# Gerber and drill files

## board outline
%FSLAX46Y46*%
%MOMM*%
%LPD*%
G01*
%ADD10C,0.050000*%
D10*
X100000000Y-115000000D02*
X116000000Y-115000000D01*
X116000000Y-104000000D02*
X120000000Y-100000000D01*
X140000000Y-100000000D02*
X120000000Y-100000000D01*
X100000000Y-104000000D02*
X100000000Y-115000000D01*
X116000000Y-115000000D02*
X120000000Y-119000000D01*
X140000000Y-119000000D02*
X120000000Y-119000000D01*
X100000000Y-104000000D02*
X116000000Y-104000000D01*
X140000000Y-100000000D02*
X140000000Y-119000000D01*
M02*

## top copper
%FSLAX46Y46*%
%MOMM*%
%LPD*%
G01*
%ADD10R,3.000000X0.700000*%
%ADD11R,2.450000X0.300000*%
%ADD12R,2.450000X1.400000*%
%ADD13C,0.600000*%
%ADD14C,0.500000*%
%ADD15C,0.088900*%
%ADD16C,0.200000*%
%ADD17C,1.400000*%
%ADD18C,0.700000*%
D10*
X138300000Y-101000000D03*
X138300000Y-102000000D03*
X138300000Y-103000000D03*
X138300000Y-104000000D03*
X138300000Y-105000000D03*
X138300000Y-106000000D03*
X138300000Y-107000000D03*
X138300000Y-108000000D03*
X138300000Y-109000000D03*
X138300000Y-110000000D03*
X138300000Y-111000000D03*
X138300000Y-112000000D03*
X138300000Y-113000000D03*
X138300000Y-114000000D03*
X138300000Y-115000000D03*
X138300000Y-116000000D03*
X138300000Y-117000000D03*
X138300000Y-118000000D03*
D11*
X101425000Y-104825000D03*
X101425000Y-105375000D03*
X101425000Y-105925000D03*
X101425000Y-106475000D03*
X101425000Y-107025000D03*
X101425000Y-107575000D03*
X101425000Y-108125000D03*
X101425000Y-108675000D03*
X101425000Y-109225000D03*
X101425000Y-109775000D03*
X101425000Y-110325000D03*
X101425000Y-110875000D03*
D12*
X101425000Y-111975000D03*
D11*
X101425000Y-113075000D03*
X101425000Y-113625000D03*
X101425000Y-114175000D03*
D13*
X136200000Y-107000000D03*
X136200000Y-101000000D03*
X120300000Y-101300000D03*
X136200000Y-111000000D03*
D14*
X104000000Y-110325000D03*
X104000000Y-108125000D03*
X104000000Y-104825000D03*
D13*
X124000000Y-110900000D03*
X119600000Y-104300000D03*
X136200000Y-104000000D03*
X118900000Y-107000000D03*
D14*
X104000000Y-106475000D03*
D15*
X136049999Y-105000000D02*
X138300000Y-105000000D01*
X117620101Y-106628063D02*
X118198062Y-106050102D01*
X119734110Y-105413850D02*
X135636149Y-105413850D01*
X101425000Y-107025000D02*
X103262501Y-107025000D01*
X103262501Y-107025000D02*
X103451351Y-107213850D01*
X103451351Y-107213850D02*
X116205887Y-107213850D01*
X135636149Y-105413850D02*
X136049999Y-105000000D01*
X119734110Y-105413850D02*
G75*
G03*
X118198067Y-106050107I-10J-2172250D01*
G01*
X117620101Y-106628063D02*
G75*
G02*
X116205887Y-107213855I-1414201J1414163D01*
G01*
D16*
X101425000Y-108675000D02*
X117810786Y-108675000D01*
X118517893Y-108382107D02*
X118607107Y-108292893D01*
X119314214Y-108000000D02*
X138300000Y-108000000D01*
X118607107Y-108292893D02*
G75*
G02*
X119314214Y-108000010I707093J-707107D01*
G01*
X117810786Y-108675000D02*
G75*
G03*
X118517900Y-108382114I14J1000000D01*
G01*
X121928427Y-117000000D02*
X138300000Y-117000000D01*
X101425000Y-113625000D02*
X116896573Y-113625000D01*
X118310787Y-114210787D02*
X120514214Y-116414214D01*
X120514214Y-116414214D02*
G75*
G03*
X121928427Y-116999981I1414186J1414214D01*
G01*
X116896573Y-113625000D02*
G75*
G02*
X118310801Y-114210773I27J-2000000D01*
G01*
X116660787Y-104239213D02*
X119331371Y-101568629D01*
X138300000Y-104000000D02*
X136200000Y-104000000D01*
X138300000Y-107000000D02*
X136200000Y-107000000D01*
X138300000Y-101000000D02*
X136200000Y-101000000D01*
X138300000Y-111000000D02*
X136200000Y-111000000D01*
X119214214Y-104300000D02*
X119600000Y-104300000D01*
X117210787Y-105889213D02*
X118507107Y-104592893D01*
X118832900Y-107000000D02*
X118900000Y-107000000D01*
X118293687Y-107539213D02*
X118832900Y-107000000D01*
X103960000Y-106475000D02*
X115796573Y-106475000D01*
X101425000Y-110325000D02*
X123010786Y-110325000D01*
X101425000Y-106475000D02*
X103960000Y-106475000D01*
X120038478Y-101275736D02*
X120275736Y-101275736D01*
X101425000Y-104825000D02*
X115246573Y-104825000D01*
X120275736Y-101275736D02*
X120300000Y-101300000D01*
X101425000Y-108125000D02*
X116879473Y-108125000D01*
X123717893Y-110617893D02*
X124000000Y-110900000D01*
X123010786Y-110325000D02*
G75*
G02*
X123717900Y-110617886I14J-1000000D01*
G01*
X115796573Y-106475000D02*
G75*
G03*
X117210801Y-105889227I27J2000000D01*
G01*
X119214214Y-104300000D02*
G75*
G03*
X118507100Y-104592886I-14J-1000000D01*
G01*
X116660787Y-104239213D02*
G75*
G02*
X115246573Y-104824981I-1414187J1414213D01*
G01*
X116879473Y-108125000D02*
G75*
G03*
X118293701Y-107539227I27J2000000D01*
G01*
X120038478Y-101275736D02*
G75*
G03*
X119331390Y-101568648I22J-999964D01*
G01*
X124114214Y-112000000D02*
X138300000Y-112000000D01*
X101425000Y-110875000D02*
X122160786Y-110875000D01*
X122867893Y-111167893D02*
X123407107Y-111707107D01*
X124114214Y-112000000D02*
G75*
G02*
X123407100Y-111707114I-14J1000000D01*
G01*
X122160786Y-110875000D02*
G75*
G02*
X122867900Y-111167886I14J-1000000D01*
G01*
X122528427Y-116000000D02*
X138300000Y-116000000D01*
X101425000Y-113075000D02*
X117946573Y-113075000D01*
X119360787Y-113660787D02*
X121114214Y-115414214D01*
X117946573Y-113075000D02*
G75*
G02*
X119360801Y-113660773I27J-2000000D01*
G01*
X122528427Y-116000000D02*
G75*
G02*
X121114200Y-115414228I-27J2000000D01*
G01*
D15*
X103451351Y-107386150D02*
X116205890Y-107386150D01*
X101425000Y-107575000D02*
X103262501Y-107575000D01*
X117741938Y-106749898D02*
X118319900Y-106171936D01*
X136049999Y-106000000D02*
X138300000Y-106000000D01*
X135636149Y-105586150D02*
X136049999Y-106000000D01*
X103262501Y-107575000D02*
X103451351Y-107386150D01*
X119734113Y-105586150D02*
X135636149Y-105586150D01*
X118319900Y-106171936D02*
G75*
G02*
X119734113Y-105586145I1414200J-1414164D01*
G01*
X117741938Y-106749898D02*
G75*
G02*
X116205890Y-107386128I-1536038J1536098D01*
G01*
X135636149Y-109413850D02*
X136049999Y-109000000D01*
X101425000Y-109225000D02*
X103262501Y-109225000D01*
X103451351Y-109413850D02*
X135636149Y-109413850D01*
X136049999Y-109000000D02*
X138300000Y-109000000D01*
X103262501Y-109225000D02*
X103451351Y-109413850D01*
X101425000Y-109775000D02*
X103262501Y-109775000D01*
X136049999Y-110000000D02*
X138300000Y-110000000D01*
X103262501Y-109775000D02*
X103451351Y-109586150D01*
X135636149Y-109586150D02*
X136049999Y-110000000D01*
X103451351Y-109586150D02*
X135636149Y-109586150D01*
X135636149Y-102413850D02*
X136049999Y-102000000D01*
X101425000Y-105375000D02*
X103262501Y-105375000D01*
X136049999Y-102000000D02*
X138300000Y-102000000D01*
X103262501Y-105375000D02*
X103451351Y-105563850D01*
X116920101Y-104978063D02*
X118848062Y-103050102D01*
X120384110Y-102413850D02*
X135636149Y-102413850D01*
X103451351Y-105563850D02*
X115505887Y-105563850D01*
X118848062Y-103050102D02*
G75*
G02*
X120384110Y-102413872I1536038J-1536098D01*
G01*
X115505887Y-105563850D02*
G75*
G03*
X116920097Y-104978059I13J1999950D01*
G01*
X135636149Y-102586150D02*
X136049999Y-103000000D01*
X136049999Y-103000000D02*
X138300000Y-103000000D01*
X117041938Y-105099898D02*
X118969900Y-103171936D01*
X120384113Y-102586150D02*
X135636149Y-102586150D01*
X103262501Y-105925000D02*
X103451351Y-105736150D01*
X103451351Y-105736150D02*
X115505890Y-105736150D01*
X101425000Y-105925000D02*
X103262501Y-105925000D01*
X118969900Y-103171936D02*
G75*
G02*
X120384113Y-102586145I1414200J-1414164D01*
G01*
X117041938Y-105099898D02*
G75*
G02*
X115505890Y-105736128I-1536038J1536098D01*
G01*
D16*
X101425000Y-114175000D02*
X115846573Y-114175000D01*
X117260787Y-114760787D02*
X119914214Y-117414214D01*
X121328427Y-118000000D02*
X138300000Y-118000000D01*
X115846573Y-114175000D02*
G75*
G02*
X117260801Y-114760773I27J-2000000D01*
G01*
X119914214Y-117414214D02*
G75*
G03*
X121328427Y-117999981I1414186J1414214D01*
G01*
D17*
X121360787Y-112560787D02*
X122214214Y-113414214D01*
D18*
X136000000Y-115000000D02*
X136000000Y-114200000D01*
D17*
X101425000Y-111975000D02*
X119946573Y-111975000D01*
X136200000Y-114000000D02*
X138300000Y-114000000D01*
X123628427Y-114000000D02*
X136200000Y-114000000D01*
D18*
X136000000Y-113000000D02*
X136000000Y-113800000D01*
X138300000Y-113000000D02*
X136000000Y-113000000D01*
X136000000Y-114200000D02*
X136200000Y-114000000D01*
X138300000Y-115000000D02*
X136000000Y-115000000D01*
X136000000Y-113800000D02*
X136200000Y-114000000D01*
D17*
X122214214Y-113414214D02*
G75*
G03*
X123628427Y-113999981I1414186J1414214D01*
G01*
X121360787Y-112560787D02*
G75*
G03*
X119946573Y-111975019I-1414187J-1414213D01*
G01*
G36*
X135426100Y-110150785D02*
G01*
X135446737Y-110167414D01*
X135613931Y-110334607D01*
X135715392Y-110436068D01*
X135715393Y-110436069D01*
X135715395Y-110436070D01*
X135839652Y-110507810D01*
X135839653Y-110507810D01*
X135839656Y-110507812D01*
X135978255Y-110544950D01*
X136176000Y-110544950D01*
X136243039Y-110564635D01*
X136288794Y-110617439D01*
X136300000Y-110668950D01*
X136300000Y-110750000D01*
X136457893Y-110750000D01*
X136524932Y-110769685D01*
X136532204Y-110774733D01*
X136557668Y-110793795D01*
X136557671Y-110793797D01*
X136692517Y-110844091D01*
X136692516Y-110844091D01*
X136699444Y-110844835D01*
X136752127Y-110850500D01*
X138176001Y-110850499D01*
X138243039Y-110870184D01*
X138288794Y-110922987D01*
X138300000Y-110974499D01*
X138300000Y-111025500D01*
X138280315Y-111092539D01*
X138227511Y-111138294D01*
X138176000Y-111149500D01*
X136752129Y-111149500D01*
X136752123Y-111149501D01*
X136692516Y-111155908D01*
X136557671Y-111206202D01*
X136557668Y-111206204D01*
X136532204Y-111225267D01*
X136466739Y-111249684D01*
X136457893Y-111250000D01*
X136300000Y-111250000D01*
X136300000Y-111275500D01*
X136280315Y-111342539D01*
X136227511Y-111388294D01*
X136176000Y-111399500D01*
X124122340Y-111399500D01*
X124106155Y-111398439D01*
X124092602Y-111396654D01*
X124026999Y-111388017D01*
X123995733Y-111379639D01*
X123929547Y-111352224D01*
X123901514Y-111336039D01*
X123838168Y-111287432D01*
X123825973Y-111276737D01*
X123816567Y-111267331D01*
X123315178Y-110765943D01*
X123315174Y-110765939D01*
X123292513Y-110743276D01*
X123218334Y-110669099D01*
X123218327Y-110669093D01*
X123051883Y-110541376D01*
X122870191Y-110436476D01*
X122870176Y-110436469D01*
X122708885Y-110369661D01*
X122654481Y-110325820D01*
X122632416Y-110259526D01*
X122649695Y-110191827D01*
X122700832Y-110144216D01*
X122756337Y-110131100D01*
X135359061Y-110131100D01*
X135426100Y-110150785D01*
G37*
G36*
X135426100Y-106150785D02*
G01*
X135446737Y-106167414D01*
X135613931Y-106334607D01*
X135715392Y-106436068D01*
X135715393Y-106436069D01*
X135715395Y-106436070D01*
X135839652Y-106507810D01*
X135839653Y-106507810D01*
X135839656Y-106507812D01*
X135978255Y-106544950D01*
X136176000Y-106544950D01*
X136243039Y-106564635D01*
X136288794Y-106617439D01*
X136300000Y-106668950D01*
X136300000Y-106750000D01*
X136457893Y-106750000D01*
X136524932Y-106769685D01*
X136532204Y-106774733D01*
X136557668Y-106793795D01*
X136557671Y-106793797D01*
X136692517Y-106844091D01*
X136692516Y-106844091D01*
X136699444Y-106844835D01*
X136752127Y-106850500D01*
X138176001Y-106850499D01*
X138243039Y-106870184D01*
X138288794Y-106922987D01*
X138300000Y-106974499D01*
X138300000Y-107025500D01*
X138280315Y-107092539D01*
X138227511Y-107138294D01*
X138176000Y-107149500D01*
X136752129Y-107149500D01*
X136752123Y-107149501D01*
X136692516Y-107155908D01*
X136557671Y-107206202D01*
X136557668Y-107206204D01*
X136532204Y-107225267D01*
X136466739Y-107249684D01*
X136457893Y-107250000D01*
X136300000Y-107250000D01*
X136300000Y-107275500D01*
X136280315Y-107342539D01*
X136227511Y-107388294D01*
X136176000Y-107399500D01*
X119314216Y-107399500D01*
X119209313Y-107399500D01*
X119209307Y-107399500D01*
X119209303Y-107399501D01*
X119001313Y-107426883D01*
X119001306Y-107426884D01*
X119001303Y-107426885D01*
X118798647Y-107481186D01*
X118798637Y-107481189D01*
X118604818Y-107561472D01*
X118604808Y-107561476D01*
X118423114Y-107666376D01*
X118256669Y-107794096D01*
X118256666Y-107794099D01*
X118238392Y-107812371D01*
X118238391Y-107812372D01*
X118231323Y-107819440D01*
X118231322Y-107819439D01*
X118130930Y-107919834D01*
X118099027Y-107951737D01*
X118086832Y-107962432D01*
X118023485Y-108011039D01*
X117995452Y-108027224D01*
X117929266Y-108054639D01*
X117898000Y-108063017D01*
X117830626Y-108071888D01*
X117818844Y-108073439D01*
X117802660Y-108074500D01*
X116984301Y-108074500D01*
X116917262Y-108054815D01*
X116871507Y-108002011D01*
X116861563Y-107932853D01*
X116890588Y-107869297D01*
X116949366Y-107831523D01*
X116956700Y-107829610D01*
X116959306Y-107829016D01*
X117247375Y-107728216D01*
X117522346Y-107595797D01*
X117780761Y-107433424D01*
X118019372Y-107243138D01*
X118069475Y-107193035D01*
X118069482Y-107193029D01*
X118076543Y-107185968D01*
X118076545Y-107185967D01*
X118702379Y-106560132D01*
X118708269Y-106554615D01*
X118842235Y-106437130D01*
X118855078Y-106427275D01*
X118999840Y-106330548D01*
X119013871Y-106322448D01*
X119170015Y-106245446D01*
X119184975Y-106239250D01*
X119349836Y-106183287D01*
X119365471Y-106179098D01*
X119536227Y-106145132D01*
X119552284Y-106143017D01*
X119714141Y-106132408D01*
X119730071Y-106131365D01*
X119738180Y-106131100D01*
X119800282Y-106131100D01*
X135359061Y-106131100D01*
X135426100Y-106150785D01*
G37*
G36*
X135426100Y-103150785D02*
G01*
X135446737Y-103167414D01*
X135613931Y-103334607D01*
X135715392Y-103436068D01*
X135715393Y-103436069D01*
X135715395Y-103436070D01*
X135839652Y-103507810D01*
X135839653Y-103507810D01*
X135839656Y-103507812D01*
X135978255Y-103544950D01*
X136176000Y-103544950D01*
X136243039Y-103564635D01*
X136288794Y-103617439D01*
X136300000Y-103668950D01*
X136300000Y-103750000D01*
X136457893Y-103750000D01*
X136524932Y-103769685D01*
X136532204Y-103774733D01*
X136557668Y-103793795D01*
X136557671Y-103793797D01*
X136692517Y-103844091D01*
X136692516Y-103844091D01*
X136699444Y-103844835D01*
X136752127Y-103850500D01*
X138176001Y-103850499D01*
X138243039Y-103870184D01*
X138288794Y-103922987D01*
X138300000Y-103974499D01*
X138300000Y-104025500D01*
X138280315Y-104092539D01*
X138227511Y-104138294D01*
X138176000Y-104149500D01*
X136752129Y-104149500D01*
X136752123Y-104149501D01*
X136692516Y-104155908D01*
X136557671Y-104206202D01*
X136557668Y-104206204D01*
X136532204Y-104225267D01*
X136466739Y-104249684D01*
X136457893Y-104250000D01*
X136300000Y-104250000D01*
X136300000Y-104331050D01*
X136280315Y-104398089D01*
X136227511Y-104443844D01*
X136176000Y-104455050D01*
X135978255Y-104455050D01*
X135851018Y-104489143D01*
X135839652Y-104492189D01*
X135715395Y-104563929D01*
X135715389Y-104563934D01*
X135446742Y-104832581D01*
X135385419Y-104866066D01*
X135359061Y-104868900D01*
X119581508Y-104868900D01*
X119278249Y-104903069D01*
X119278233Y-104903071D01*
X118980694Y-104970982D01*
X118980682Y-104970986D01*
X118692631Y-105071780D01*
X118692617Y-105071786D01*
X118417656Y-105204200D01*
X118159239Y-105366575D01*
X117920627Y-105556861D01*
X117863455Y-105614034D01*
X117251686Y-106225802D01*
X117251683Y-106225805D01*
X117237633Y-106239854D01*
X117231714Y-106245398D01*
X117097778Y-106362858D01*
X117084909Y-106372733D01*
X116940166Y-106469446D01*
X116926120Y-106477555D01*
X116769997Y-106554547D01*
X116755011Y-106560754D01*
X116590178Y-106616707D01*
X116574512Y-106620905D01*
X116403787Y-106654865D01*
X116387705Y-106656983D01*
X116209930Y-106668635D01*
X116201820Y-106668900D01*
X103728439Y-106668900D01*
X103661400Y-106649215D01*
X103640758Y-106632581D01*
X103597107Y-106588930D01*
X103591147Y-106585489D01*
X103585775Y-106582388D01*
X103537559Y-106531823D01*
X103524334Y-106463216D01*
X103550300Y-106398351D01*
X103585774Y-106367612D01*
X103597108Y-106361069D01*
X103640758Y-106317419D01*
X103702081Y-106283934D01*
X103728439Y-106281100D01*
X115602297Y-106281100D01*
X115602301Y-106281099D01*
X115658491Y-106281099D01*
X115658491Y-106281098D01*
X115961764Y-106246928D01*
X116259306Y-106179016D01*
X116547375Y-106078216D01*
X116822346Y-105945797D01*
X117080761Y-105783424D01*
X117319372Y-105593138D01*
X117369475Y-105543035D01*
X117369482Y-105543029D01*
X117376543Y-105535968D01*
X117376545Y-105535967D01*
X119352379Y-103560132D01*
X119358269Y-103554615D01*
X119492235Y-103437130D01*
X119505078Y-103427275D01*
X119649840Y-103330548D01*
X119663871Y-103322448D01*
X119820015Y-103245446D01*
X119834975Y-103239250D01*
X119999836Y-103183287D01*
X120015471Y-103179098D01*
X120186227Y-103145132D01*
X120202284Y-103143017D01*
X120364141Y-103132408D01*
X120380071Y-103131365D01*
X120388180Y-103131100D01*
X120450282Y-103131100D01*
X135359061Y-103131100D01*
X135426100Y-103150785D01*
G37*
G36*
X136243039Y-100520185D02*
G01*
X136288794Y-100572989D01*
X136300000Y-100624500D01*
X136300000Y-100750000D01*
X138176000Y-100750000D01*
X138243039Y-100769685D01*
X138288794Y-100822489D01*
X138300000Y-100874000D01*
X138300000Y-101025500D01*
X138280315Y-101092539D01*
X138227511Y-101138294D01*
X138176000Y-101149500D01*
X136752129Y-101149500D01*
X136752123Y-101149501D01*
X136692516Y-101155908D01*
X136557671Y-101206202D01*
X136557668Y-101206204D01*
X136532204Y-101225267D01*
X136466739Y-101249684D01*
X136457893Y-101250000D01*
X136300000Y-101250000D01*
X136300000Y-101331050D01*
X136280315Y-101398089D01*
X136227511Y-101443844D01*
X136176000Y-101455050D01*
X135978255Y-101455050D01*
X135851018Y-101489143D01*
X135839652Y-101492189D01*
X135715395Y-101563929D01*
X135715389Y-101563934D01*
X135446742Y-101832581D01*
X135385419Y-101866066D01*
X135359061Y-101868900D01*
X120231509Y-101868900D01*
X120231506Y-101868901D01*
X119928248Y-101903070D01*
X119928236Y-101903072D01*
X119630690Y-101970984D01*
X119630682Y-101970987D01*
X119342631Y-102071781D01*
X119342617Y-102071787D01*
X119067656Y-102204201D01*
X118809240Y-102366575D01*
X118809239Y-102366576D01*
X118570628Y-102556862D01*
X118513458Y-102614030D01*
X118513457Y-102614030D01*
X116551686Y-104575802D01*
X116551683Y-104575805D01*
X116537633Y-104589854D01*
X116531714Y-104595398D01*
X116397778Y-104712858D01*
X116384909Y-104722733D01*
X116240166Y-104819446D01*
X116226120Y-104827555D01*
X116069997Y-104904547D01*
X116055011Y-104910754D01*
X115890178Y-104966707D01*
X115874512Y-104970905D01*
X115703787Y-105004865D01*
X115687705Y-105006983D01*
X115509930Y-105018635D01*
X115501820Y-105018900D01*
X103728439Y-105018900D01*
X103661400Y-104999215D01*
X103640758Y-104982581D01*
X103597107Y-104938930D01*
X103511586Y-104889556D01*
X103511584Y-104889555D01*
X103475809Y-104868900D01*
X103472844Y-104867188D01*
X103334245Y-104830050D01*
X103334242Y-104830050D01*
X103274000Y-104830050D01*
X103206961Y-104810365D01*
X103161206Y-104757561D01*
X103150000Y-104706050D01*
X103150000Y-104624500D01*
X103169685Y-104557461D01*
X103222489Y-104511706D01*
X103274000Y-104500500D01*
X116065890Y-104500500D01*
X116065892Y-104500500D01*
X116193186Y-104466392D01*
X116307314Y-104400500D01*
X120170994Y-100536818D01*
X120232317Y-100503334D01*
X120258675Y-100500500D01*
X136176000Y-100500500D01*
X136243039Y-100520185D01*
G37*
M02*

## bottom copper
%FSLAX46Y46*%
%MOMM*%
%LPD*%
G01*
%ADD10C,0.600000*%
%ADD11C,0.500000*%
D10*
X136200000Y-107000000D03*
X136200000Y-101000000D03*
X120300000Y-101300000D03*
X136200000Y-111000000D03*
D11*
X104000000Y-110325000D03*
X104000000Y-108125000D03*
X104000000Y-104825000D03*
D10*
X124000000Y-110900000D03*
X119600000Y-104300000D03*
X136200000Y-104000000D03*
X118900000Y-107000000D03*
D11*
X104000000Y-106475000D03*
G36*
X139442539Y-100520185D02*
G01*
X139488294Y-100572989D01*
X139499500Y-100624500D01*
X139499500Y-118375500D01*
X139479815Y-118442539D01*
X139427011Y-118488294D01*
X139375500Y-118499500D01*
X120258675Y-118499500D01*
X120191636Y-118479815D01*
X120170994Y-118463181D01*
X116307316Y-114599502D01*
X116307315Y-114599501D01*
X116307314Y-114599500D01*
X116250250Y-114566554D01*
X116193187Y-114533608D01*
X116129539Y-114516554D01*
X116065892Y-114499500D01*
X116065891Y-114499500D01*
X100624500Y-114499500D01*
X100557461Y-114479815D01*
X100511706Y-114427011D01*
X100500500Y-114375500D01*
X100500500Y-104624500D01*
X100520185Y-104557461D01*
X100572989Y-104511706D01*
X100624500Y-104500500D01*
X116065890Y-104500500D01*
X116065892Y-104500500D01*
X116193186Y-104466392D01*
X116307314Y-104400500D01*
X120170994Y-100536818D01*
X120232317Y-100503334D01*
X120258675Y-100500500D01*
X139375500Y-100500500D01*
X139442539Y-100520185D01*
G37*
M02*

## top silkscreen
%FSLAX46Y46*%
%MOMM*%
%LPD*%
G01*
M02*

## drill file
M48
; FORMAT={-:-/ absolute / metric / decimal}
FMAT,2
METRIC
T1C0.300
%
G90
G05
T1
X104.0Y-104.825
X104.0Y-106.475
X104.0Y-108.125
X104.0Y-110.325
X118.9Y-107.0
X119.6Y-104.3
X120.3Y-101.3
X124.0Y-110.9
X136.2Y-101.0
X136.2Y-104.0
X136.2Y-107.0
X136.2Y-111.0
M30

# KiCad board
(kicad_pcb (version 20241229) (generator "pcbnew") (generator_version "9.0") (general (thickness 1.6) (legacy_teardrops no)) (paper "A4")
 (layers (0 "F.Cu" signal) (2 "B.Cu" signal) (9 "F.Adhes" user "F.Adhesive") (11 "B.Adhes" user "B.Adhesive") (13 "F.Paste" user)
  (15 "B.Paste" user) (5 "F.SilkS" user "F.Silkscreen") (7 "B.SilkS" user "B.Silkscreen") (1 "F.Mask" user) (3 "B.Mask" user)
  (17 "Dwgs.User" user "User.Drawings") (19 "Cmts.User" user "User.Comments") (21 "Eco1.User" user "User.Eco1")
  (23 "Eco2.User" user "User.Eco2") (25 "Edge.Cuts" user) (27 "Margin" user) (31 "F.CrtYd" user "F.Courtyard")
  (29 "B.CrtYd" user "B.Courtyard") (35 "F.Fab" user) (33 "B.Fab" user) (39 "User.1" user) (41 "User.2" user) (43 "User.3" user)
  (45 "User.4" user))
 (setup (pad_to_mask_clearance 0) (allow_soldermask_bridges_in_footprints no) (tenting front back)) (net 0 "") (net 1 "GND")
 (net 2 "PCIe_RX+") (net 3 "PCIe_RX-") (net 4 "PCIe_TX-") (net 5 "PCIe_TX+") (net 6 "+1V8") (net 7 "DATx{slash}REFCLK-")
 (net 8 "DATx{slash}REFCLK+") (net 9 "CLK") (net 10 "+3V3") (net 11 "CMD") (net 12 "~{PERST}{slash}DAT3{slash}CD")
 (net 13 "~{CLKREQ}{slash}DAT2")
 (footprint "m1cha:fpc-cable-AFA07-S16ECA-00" (layer "F.Cu") (at 138.3 109.5 -90)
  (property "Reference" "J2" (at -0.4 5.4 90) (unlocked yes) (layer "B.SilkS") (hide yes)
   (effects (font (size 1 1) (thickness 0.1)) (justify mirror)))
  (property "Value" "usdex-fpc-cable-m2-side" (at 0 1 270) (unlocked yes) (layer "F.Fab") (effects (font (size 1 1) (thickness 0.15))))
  (pad "1" smd rect (at -8.5 0 270) (size 0.7 3) (layers "F.Cu" "F.Mask" "F.Paste") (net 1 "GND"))
  (pad "2" smd rect (at -7.5 0 270) (size 0.7 3) (layers "F.Cu" "F.Mask" "F.Paste") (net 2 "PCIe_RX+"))
  (pad "3" smd rect (at -6.5 0 270) (size 0.7 3) (layers "F.Cu" "F.Mask" "F.Paste") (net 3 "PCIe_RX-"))
  (pad "4" smd rect (at -5.5 0 270) (size 0.7 3) (layers "F.Cu" "F.Mask" "F.Paste") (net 1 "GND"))
  (pad "5" smd rect (at -4.5 0 270) (size 0.7 3) (layers "F.Cu" "F.Mask" "F.Paste") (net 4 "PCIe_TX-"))
  (pad "6" smd rect (at -3.5 0 270) (size 0.7 3) (layers "F.Cu" "F.Mask" "F.Paste") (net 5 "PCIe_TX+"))
  (pad "7" smd rect (at -2.5 0 270) (size 0.7 3) (layers "F.Cu" "F.Mask" "F.Paste") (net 1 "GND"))
  (pad "8" smd rect (at -1.5 0 270) (size 0.7 3) (layers "F.Cu" "F.Mask" "F.Paste") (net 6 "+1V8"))
  (pad "9" smd rect (at -0.5 0 270) (size 0.7 3) (layers "F.Cu" "F.Mask" "F.Paste") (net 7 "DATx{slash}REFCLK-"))
  (pad "10" smd rect (at 0.5 0 270) (size 0.7 3) (layers "F.Cu" "F.Mask" "F.Paste") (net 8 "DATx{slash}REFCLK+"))
  (pad "11" smd rect (at 1.5 0 270) (size 0.7 3) (layers "F.Cu" "F.Mask" "F.Paste") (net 1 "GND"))
  (pad "12" smd rect (at 2.5 0 270) (size 0.7 3) (layers "F.Cu" "F.Mask" "F.Paste") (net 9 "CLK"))
  (pad "13" smd rect (at 3.5 0 270) (size 0.7 3) (layers "F.Cu" "F.Mask" "F.Paste") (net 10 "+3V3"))
  (pad "14" smd rect (at 4.5 0 270) (size 0.7 3) (layers "F.Cu" "F.Mask" "F.Paste") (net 10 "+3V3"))
  (pad "15" smd rect (at 5.5 0 270) (size 0.7 3) (layers "F.Cu" "F.Mask" "F.Paste") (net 10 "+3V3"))
  (pad "16" smd rect (at 6.5 0 270) (size 0.7 3) (layers "F.Cu" "F.Mask" "F.Paste") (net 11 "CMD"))
  (pad "17" smd rect (at 7.5 0 270) (size 0.7 3) (layers "F.Cu" "F.Mask" "F.Paste") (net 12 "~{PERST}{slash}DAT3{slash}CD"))
  (pad "18" smd rect (at 8.5 0 270) (size 0.7 3) (layers "F.Cu" "F.Mask" "F.Paste") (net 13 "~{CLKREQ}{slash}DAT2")))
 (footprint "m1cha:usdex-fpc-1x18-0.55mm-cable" (layer "F.Cu") (at 101.425 109.5 -90)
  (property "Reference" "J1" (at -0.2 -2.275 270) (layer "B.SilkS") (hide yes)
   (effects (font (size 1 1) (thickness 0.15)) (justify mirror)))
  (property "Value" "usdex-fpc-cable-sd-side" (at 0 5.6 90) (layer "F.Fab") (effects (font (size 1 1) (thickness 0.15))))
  (pad "1" smd rect (at -4.675 0 270) (size 0.3 2.45) (layers "F.Cu" "F.Mask" "F.Paste") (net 1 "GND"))
  (pad "2" smd rect (at -4.125 0 270) (size 0.3 2.45) (layers "F.Cu" "F.Mask" "F.Paste") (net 2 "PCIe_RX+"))
  (pad "3" smd rect (at -3.575 0 270) (size 0.3 2.45) (layers "F.Cu" "F.Mask" "F.Paste") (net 3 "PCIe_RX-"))
  (pad "4" smd rect (at -3.025 0 270) (size 0.3 2.45) (layers "F.Cu" "F.Mask" "F.Paste") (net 1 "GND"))
  (pad "5" smd rect (at -2.475 0 270) (size 0.3 2.45) (layers "F.Cu" "F.Mask" "F.Paste") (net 4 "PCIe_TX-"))
  (pad "6" smd rect (at -1.925 0 270) (size 0.3 2.45) (layers "F.Cu" "F.Mask" "F.Paste") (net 5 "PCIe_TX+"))
  (pad "7" smd rect (at -1.375 0 270) (size 0.3 2.45) (layers "F.Cu" "F.Mask" "F.Paste") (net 1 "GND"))
  (pad "8" smd rect (at -0.825 0 270) (size 0.3 2.45) (layers "F.Cu" "F.Mask" "F.Paste") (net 6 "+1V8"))
  (pad "9" smd rect (at -0.275 0 270) (size 0.3 2.45) (layers "F.Cu" "F.Mask" "F.Paste") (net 7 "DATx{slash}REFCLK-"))
  (pad "10" smd rect (at 0.275 0 270) (size 0.3 2.45) (layers "F.Cu" "F.Mask" "F.Paste") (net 8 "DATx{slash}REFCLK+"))
  (pad "11" smd rect (at 0.825 0 270) (size 0.3 2.45) (layers "F.Cu" "F.Mask" "F.Paste") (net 1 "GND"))
  (pad "12" smd rect (at 1.375 0 270) (size 0.3 2.45) (layers "F.Cu" "F.Mask" "F.Paste") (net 9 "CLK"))
  (pad "13" smd rect (at 2.475 0 270) (size 1.4 2.45) (layers "F.Cu" "F.Mask" "F.Paste") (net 10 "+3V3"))
  (pad "14" smd rect (at 3.575 0 270) (size 0.3 2.45) (layers "F.Cu" "F.Mask" "F.Paste") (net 11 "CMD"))
  (pad "15" smd rect (at 4.125 0 270) (size 0.3 2.45) (layers "F.Cu" "F.Mask" "F.Paste") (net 12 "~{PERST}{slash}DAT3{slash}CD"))
  (pad "16" smd rect (at 4.675 0 270) (size 0.3 2.45) (layers "F.Cu" "F.Mask" "F.Paste") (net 13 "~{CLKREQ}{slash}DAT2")))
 (gr_line (start 100 115) (end 116 115) (stroke (width 0.05) (type solid)) (layer "Edge.Cuts"))
 (gr_line (start 116 104) (end 120 100) (stroke (width 0.05) (type default)) (layer "Edge.Cuts"))
 (gr_line (start 140 100) (end 120 100) (stroke (width 0.05) (type solid)) (layer "Edge.Cuts"))
 (gr_line (start 100 104) (end 100 115) (stroke (width 0.05) (type solid)) (layer "Edge.Cuts"))
 (gr_line (start 116 115) (end 120 119) (stroke (width 0.05) (type default)) (layer "Edge.Cuts"))
 (gr_line (start 140 119) (end 120 119) (stroke (width 0.05) (type solid)) (layer "Edge.Cuts"))
 (gr_line (start 100 104) (end 116 104) (stroke (width 0.05) (type solid)) (layer "Edge.Cuts"))
 (gr_line (start 140 100) (end 140 119) (stroke (width 0.05) (type default)) (layer "Edge.Cuts"))
 (segment (start 136.049999 105) (end 138.3 105) (width 0.0889) (layer "F.Cu") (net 4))
 (segment (start 117.620101 106.628063) (end 118.198062 106.050102) (width 0.0889) (layer "F.Cu") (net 4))
 (segment (start 119.73411 105.41385) (end 135.636149 105.41385) (width 0.0889) (layer "F.Cu") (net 4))
 (segment (start 101.425 107.025) (end 103.262501 107.025) (width 0.0889) (layer "F.Cu") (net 4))
 (segment (start 103.262501 107.025) (end 103.451351 107.21385) (width 0.0889) (layer "F.Cu") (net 4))
 (segment (start 103.451351 107.21385) (end 116.205887 107.21385) (width 0.0889) (layer "F.Cu") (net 4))
 (segment (start 135.636149 105.41385) (end 136.049999 105) (width 0.0889) (layer "F.Cu") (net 4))
 (arc (start 119.73411 105.41385) (mid 118.902807 105.579206) (end 118.198062 106.050102) (width 0.0889) (layer "F.Cu") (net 4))
 (arc (start 117.620101 106.628063) (mid 116.971254 107.061609) (end 116.205887 107.21385) (width 0.0889) (layer "F.Cu") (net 4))
 (segment (start 101.425 108.675) (end 117.810786 108.675) (width 0.2) (layer "F.Cu") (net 6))
 (segment (start 118.517893 108.382107) (end 118.607107 108.292893) (width 0.2) (layer "F.Cu") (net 6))
 (segment (start 119.314214 108) (end 138.3 108) (width 0.2) (layer "F.Cu") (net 6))
 (arc (start 118.607107 108.292893) (mid 118.93153 108.07612) (end 119.314214 108) (width 0.2) (layer "F.Cu") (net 6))
 (arc (start 117.810786 108.675) (mid 118.193469 108.59888) (end 118.517893 108.382107) (width 0.2) (layer "F.Cu") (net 6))
 (segment (start 121.928427 117) (end 138.3 117) (width 0.2) (layer "F.Cu") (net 12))
 (segment (start 101.425 113.625) (end 116.896573 113.625) (width 0.2) (layer "F.Cu") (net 12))
 (segment (start 118.310787 114.210787) (end 120.514214 116.414214) (width 0.2) (layer "F.Cu") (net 12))
 (arc (start 120.514214 116.414214) (mid 121.16306 116.847759) (end 121.928427 117) (width 0.2) (layer "F.Cu") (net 12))
 (arc (start 116.896573 113.625) (mid 117.66194 113.777241) (end 118.310787 114.210787) (width 0.2) (layer "F.Cu") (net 12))
 (segment (start 116.660787 104.239213) (end 119.331371 101.568629) (width 0.2) (layer "F.Cu") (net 1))
 (segment (start 138.3 104) (end 136.2 104) (width 0.2) (layer "F.Cu") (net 1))
 (segment (start 138.3 107) (end 136.2 107) (width 0.2) (layer "F.Cu") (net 1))
 (segment (start 138.3 101) (end 136.2 101) (width 0.2) (layer "F.Cu") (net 1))
 (segment (start 138.3 111) (end 136.2 111) (width 0.2) (layer "F.Cu") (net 1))
 (segment (start 119.214214 104.3) (end 119.6 104.3) (width 0.2) (layer "F.Cu") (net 1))
 (segment (start 117.210787 105.889213) (end 118.507107 104.592893) (width 0.2) (layer "F.Cu") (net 1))
 (segment (start 118.8329 107) (end 118.9 107) (width 0.2) (layer "F.Cu") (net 1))
 (segment (start 118.293687 107.539213) (end 118.8329 107) (width 0.2) (layer "F.Cu") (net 1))
 (segment (start 103.96 106.475) (end 115.796573 106.475) (width 0.2) (layer "F.Cu") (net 1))
 (segment (start 101.425 110.325) (end 123.010786 110.325) (width 0.2) (layer "F.Cu") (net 1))
 (segment (start 101.425 106.475) (end 103.96 106.475) (width 0.2) (layer "F.Cu") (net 1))
 (segment (start 120.038478 101.275736) (end 120.275736 101.275736) (width 0.2) (layer "F.Cu") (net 1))
 (segment (start 101.425 104.825) (end 115.246573 104.825) (width 0.2) (layer "F.Cu") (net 1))
 (segment (start 120.275736 101.275736) (end 120.3 101.3) (width 0.2) (layer "F.Cu") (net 1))
 (segment (start 101.425 108.125) (end 116.879473 108.125) (width 0.2) (layer "F.Cu") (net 1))
 (segment (start 123.717893 110.617893) (end 124 110.9) (width 0.2) (layer "F.Cu") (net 1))
 (via (at 136.2 107) (size 0.6) (drill 0.3) (layers "F.Cu" "B.Cu") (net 1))
 (via (at 136.2 101) (size 0.6) (drill 0.3) (layers "F.Cu" "B.Cu") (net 1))
 (via (at 120.3 101.3) (size 0.6) (drill 0.3) (layers "F.Cu" "B.Cu") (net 1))
 (via (at 136.2 111) (size 0.6) (drill 0.3) (layers "F.Cu" "B.Cu") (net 1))
 (via (at 104 110.325) (size 0.5) (drill 0.3) (layers "F.Cu" "B.Cu") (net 1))
 (via (at 104 108.125) (size 0.5) (drill 0.3) (layers "F.Cu" "B.Cu") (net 1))
 (via (at 104 104.825) (size 0.5) (drill 0.3) (layers "F.Cu" "B.Cu") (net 1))
 (via (at 124 110.9) (size 0.6) (drill 0.3) (layers "F.Cu" "B.Cu") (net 1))
 (via (at 119.6 104.3) (size 0.6) (drill 0.3) (layers "F.Cu" "B.Cu") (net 1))
 (via (at 136.2 104) (size 0.6) (drill 0.3) (layers "F.Cu" "B.Cu") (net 1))
 (via (at 118.9 107) (size 0.6) (drill 0.3) (layers "F.Cu" "B.Cu") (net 1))
 (via (at 104 106.475) (size 0.5) (drill 0.3) (layers "F.Cu" "B.Cu") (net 1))
 (arc (start 123.010786 110.325) (mid 123.393469 110.40112) (end 123.717893 110.617893) (width 0.2) (layer "F.Cu") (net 1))
 (arc (start 115.796573 106.475) (mid 116.56194 106.322759) (end 117.210787 105.889213) (width 0.2) (layer "F.Cu") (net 1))
 (arc (start 119.214214 104.3) (mid 118.831531 104.37612) (end 118.507107 104.592893) (width 0.2) (layer "F.Cu") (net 1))
 (arc (start 116.660787 104.239213) (mid 116.01194 104.672759) (end 115.246573 104.825) (width 0.2) (layer "F.Cu") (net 1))
 (arc (start 116.879473 108.125) (mid 117.64484 107.972759) (end 118.293687 107.539213) (width 0.2) (layer "F.Cu") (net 1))
 (arc (start 120.038478 101.275736) (mid 119.655795 101.351856) (end 119.331371 101.568629) (width 0.2) (layer "F.Cu") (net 1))
 (segment (start 124.114214 112) (end 138.3 112) (width 0.2) (layer "F.Cu") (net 9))
 (segment (start 101.425 110.875) (end 122.160786 110.875) (width 0.2) (layer "F.Cu") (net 9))
 (segment (start 122.867893 111.167893) (end 123.407107 111.707107) (width 0.2) (layer "F.Cu") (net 9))
 (arc (start 124.114214 112) (mid 123.731531 111.92388) (end 123.407107 111.707107) (width 0.2) (layer "F.Cu") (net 9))
 (arc (start 122.160786 110.875) (mid 122.543469 110.95112) (end 122.867893 111.167893) (width 0.2) (layer "F.Cu") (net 9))
 (segment (start 122.528427 116) (end 138.3 116) (width 0.2) (layer "F.Cu") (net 11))
 (segment (start 101.425 113.075) (end 117.946573 113.075) (width 0.2) (layer "F.Cu") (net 11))
 (segment (start 119.360787 113.660787) (end 121.114214 115.414214) (width 0.2) (layer "F.Cu") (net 11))
 (arc (start 117.946573 113.075) (mid 118.71194 113.227241) (end 119.360787 113.660787) (width 0.2) (layer "F.Cu") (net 11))
 (arc (start 122.528427 116) (mid 121.76306 115.847759) (end 121.114214 115.414214) (width 0.2) (layer "F.Cu") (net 11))
 (segment (start 103.451351 107.38615) (end 116.20589 107.38615) (width 0.0889) (layer "F.Cu") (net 5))
 (segment (start 101.425 107.575) (end 103.262501 107.575) (width 0.0889) (layer "F.Cu") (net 5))
 (segment (start 117.741938 106.749898) (end 118.3199 106.171936) (width 0.0889) (layer "F.Cu") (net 5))
 (segment (start 136.049999 106) (end 138.3 106) (width 0.0889) (layer "F.Cu") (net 5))
 (segment (start 135.636149 105.58615) (end 136.049999 106) (width 0.0889) (layer "F.Cu") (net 5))
 (segment (start 103.262501 107.575) (end 103.451351 107.38615) (width 0.0889) (layer "F.Cu") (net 5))
 (segment (start 119.734113 105.58615) (end 135.636149 105.58615) (width 0.0889) (layer "F.Cu") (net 5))
 (arc (start 118.3199 106.171936) (mid 118.968746 105.738391) (end 119.734113 105.58615) (width 0.0889) (layer "F.Cu") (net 5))
 (arc (start 117.741938 106.749898) (mid 117.037193 107.220793) (end 116.20589 107.38615) (width 0.0889) (layer "F.Cu") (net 5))
 (segment (start 135.636149 109.41385) (end 136.049999 109) (width 0.0889) (layer "F.Cu") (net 7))
 (segment (start 101.425 109.225) (end 103.262501 109.225) (width 0.0889) (layer "F.Cu") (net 7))
 (segment (start 103.451351 109.41385) (end 135.636149 109.41385) (width 0.0889) (layer "F.Cu") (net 7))
 (segment (start 136.049999 109) (end 138.3 109) (width 0.0889) (layer "F.Cu") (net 7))
 (segment (start 103.262501 109.225) (end 103.451351 109.41385) (width 0.0889) (layer "F.Cu") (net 7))
 (segment (start 101.425 109.775) (end 103.262501 109.775) (width 0.0889) (layer "F.Cu") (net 8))
 (segment (start 136.049999 110) (end 138.3 110) (width 0.0889) (layer "F.Cu") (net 8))
 (segment (start 103.262501 109.775) (end 103.451351 109.58615) (width 0.0889) (layer "F.Cu") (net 8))
 (segment (start 135.636149 109.58615) (end 136.049999 110) (width 0.0889) (layer "F.Cu") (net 8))
 (segment (start 103.451351 109.58615) (end 135.636149 109.58615) (width 0.0889) (layer "F.Cu") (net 8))
 (segment (start 135.636149 102.41385) (end 136.049999 102) (width 0.0889) (layer "F.Cu") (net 2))
 (segment (start 101.425 105.375) (end 103.262501 105.375) (width 0.0889) (layer "F.Cu") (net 2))
 (segment (start 136.049999 102) (end 138.3 102) (width 0.0889) (layer "F.Cu") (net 2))
 (segment (start 103.262501 105.375) (end 103.451351 105.56385) (width 0.0889) (layer "F.Cu") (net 2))
 (segment (start 116.920101 104.978063) (end 118.848062 103.050102) (width 0.0889) (layer "F.Cu") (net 2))
 (segment (start 120.38411 102.41385) (end 135.636149 102.41385) (width 0.0889) (layer "F.Cu") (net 2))
 (segment (start 103.451351 105.56385) (end 115.505887 105.56385) (width 0.0889) (layer "F.Cu") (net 2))
 (arc (start 118.848062 103.050102) (mid 119.552807 102.579207) (end 120.38411 102.41385) (width 0.0889) (layer "F.Cu") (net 2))
 (arc (start 115.505887 105.56385) (mid 116.271254 105.411609) (end 116.920101 104.978063) (width 0.0889) (layer "F.Cu") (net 2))
 (segment (start 135.636149 102.58615) (end 136.049999 103) (width 0.0889) (layer "F.Cu") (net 3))
 (segment (start 136.049999 103) (end 138.3 103) (width 0.0889) (layer "F.Cu") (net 3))
 (segment (start 117.041938 105.099898) (end 118.9699 103.171936) (width 0.0889) (layer "F.Cu") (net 3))
 (segment (start 120.384113 102.58615) (end 135.636149 102.58615) (width 0.0889) (layer "F.Cu") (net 3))
 (segment (start 103.262501 105.925) (end 103.451351 105.73615) (width 0.0889) (layer "F.Cu") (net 3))
 (segment (start 103.451351 105.73615) (end 115.50589 105.73615) (width 0.0889) (layer "F.Cu") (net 3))
 (segment (start 101.425 105.925) (end 103.262501 105.925) (width 0.0889) (layer "F.Cu") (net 3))
 (arc (start 118.9699 103.171936) (mid 119.618746 102.738391) (end 120.384113 102.58615) (width 0.0889) (layer "F.Cu") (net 3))
 (arc (start 117.041938 105.099898) (mid 116.337193 105.570793) (end 115.50589 105.73615) (width 0.0889) (layer "F.Cu") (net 3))
 (segment (start 101.425 114.175) (end 115.846573 114.175) (width 0.2) (layer "F.Cu") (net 13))
 (segment (start 117.260787 114.760787) (end 119.914214 117.414214) (width 0.2) (layer "F.Cu") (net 13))
 (segment (start 121.328427 118) (end 138.3 118) (width 0.2) (layer "F.Cu") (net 13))
 (arc (start 115.846573 114.175) (mid 116.61194 114.327241) (end 117.260787 114.760787) (width 0.2) (layer "F.Cu") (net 13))
 (arc (start 119.914214 117.414214) (mid 120.56306 117.847759) (end 121.328427 118) (width 0.2) (layer "F.Cu") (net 13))
 (segment (start 121.360787 112.560787) (end 122.214214 113.414214) (width 1.4) (layer "F.Cu") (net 10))
 (segment (start 136 115) (end 136 114.2) (width 0.7) (layer "F.Cu") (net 10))
 (segment (start 101.425 111.975) (end 119.946573 111.975) (width 1.4) (layer "F.Cu") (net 10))
 (segment (start 136.2 114) (end 138.3 114) (width 1.4) (layer "F.Cu") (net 10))
 (segment (start 123.628427 114) (end 136.2 114) (width 1.4) (layer "F.Cu") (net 10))
 (segment (start 136 113) (end 136 113.8) (width 0.7) (layer "F.Cu") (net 10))
 (segment (start 138.3 113) (end 136 113) (width 0.7) (layer "F.Cu") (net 10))
 (segment (start 136 114.2) (end 136.2 114) (width 0.7) (layer "F.Cu") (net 10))
 (segment (start 138.3 115) (end 136 115) (width 0.7) (layer "F.Cu") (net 10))
 (segment (start 136 113.8) (end 136.2 114) (width 0.7) (layer "F.Cu") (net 10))
 (arc (start 122.214214 113.414214) (mid 122.86306 113.847759) (end 123.628427 114) (width 1.4) (layer "F.Cu") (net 10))
 (arc (start 121.360787 112.560787) (mid 120.71194 112.127241) (end 119.946573 111.975) (width 1.4) (layer "F.Cu") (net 10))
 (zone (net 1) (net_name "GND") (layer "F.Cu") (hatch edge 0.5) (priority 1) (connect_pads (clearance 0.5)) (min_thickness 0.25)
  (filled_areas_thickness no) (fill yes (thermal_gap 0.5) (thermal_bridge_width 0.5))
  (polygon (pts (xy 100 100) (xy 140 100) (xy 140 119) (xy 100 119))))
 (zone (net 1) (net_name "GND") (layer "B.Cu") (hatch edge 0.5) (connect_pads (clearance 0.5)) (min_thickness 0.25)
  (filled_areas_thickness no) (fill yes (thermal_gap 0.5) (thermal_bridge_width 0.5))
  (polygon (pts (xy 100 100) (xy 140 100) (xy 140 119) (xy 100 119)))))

